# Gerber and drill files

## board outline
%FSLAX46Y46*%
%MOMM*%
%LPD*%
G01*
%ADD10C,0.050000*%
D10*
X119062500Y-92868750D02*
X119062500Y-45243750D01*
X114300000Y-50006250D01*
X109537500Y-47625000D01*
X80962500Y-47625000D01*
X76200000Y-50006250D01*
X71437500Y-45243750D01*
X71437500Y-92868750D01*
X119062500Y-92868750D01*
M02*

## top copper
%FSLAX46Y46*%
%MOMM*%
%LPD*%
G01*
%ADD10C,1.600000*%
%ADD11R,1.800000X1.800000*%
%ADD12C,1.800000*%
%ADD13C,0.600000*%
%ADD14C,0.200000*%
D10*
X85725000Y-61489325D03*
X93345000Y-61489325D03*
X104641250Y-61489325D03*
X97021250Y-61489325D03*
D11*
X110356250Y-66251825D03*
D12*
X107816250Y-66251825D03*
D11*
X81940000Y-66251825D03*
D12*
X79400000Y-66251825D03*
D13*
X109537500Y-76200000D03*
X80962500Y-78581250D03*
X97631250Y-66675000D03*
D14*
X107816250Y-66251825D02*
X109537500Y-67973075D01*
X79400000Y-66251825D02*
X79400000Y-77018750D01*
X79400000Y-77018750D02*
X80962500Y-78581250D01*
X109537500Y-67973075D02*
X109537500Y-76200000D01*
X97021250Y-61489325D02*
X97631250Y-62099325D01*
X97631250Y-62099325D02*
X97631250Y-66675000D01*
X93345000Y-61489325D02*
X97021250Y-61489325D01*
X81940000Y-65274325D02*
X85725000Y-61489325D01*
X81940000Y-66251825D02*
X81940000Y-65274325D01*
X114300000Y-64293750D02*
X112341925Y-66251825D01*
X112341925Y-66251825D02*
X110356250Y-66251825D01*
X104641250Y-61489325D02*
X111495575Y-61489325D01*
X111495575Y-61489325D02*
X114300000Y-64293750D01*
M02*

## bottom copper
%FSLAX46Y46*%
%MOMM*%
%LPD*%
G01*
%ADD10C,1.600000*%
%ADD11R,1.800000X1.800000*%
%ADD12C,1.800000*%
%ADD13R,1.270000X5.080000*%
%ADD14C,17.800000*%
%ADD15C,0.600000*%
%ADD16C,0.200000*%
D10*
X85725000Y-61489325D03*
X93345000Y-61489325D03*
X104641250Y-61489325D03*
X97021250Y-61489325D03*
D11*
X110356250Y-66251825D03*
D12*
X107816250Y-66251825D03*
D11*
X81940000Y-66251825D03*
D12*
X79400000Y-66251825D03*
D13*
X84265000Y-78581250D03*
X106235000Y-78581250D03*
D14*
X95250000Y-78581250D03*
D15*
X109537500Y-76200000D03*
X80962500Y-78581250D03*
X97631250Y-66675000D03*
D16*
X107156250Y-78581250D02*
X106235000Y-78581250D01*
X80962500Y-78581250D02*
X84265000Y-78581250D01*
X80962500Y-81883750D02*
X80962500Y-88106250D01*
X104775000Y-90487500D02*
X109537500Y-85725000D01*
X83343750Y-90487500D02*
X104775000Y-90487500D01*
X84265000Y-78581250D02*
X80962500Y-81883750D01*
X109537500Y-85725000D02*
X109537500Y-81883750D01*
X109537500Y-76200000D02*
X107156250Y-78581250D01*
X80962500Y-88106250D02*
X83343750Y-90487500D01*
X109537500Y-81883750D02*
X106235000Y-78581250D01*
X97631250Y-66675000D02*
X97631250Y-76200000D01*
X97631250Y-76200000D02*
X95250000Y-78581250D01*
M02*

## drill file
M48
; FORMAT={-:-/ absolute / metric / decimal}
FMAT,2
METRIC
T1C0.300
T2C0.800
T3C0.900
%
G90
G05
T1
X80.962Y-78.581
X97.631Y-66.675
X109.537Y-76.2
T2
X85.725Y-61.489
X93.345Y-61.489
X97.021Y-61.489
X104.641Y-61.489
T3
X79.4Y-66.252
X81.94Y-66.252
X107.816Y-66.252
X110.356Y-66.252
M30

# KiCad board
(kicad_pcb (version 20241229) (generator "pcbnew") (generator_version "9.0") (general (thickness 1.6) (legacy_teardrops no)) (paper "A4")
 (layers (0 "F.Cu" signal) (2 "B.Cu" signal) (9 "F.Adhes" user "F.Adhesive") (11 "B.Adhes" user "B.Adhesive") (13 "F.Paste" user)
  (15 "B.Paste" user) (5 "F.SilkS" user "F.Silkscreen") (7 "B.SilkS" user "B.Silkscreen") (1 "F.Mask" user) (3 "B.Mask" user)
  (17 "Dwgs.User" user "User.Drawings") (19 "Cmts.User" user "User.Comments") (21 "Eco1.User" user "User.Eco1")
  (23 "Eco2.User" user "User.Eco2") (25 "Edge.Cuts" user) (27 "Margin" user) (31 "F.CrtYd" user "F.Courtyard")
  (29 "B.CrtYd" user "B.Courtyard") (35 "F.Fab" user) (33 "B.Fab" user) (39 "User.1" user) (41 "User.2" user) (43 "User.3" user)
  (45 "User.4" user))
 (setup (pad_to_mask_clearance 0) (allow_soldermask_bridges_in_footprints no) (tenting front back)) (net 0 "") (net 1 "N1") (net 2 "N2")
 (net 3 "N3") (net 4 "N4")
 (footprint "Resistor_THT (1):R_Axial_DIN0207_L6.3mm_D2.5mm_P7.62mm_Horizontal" (layer "F.Cu") (at 85.725 61.489325)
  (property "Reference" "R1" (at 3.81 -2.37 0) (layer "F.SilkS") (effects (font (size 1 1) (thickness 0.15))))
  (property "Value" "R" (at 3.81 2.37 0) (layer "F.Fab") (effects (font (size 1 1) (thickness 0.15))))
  (pad "1" thru_hole circle (at 0 0) (size 1.6 1.6) (drill 0.8) (layers "*.Cu" "*.Mask") (remove_unused_layers no) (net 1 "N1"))
  (pad "2" thru_hole circle (at 7.62 0) (size 1.6 1.6) (drill 0.8) (layers "*.Cu" "*.Mask") (remove_unused_layers no) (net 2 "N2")))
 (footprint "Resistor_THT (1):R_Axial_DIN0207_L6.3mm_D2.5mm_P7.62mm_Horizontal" (layer "F.Cu") (at 104.64125 61.489325 180)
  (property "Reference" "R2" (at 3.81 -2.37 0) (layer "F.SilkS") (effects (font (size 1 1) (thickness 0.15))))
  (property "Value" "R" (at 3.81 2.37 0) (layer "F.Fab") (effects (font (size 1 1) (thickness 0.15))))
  (pad "1" thru_hole circle (at 0 0 180) (size 1.6 1.6) (drill 0.8) (layers "*.Cu" "*.Mask") (remove_unused_layers no) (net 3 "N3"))
  (pad "2" thru_hole circle (at 7.62 0 180) (size 1.6 1.6) (drill 0.8) (layers "*.Cu" "*.Mask") (remove_unused_layers no) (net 2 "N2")))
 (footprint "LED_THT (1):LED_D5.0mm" (layer "F.Cu") (at 110.35625 66.251825 180)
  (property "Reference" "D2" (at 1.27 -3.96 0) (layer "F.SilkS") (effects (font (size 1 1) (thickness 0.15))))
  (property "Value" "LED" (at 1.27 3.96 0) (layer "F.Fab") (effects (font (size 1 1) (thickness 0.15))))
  (pad "1" thru_hole rect (at 0 0 180) (size 1.8 1.8) (drill 0.9) (layers "*.Cu" "*.Mask") (remove_unused_layers no) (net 3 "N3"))
  (pad "2" thru_hole circle (at 2.54 0 180) (size 1.8 1.8) (drill 0.9) (layers "*.Cu" "*.Mask") (remove_unused_layers no) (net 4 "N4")))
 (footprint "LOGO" (layer "F.Cu") (at 95.25 78.58125)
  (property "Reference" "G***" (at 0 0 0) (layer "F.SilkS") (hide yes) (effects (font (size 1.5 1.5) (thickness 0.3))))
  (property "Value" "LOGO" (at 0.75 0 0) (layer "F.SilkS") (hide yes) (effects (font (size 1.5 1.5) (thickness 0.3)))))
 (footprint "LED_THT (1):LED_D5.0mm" (layer "F.Cu") (at 81.94 66.251825 180)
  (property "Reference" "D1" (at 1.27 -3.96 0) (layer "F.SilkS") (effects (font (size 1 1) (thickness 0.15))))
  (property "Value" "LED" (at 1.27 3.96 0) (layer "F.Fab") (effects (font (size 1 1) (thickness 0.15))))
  (pad "1" thru_hole rect (at 0 0 180) (size 1.8 1.8) (drill 0.9) (layers "*.Cu" "*.Mask") (remove_unused_layers no) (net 1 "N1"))
  (pad "2" thru_hole circle (at 2.54 0 180) (size 1.8 1.8) (drill 0.9) (layers "*.Cu" "*.Mask") (remove_unused_layers no) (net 4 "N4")))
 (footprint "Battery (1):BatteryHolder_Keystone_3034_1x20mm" (layer "B.Cu") (at 95.25 78.58125)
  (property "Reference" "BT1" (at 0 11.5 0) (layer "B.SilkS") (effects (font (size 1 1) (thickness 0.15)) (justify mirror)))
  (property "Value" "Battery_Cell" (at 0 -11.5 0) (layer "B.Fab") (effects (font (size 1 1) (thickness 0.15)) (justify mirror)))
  (pad "1" smd rect (at -10.985 0) (size 1.27 5.08) (layers "B.Cu" "B.Mask" "B.Paste") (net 4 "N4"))
  (pad "1" smd rect (at 10.985 0) (size 1.27 5.08) (layers "B.Cu" "B.Mask" "B.Paste") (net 4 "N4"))
  (pad "2" smd circle (at 0 0) (size 17.8 17.8) (layers "B.Cu" "B.Mask") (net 2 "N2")))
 (gr_poly
  (pts (xy 119.0625 92.86875) (xy 119.0625 45.24375) (xy 114.3 50.00625) (xy 109.5375 47.625) (xy 80.9625 47.625) (xy 76.2 50.00625)
   (xy 71.4375 45.24375) (xy 71.4375 92.86875))
  (stroke (width 0.05) (type solid)) (fill no) (layer "Edge.Cuts"))
 (segment (start 107.81625 66.251825) (end 109.5375 67.973075) (width 0.2) (layer "F.Cu") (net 4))
 (segment (start 79.4 66.251825) (end 79.4 77.01875) (width 0.2) (layer "F.Cu") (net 4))
 (segment (start 79.4 77.01875) (end 80.9625 78.58125) (width 0.2) (layer "F.Cu") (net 4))
 (segment (start 109.5375 67.973075) (end 109.5375 76.2) (width 0.2) (layer "F.Cu") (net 4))
 (via (at 109.5375 76.2) (size 0.6) (drill 0.3) (layers "F.Cu" "B.Cu") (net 4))
 (via (at 80.9625 78.58125) (size 0.6) (drill 0.3) (layers "F.Cu" "B.Cu") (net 4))
 (segment (start 107.15625 78.58125) (end 106.235 78.58125) (width 0.2) (layer "B.Cu") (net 4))
 (segment (start 80.9625 78.58125) (end 84.265 78.58125) (width 0.2) (layer "B.Cu") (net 4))
 (segment (start 80.9625 81.88375) (end 80.9625 88.10625) (width 0.2) (layer "B.Cu") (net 4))
 (segment (start 104.775 90.4875) (end 109.5375 85.725) (width 0.2) (layer "B.Cu") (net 4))
 (segment (start 83.34375 90.4875) (end 104.775 90.4875) (width 0.2) (layer "B.Cu") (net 4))
 (segment (start 84.265 78.58125) (end 80.9625 81.88375) (width 0.2) (layer "B.Cu") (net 4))
 (segment (start 109.5375 85.725) (end 109.5375 81.88375) (width 0.2) (layer "B.Cu") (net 4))
 (segment (start 109.5375 76.2) (end 107.15625 78.58125) (width 0.2) (layer "B.Cu") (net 4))
 (segment (start 80.9625 88.10625) (end 83.34375 90.4875) (width 0.2) (layer "B.Cu") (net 4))
 (segment (start 109.5375 81.88375) (end 106.235 78.58125) (width 0.2) (layer "B.Cu") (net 4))
 (segment (start 97.02125 61.489325) (end 97.63125 62.099325) (width 0.2) (layer "F.Cu") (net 2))
 (segment (start 97.63125 62.099325) (end 97.63125 66.675) (width 0.2) (layer "F.Cu") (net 2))
 (segment (start 93.345 61.489325) (end 97.02125 61.489325) (width 0.2) (layer "F.Cu") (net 2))
 (via (at 97.63125 66.675) (size 0.6) (drill 0.3) (layers "F.Cu" "B.Cu") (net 2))
 (segment (start 97.63125 66.675) (end 97.63125 76.2) (width 0.2) (layer "B.Cu") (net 2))
 (segment (start 97.63125 76.2) (end 95.25 78.58125) (width 0.2) (layer "B.Cu") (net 2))
 (segment (start 81.94 65.274325) (end 85.725 61.489325) (width 0.2) (layer "F.Cu") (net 1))
 (segment (start 81.94 66.251825) (end 81.94 65.274325) (width 0.2) (layer "F.Cu") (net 1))
 (segment (start 114.3 64.29375) (end 112.341925 66.251825) (width 0.2) (layer "F.Cu") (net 3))
 (segment (start 112.341925 66.251825) (end 110.35625 66.251825) (width 0.2) (layer "F.Cu") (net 3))
 (segment (start 104.64125 61.489325) (end 111.495575 61.489325) (width 0.2) (layer "F.Cu") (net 3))
 (segment (start 111.495575 61.489325) (end 114.3 64.29375) (width 0.2) (layer "F.Cu") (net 3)))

